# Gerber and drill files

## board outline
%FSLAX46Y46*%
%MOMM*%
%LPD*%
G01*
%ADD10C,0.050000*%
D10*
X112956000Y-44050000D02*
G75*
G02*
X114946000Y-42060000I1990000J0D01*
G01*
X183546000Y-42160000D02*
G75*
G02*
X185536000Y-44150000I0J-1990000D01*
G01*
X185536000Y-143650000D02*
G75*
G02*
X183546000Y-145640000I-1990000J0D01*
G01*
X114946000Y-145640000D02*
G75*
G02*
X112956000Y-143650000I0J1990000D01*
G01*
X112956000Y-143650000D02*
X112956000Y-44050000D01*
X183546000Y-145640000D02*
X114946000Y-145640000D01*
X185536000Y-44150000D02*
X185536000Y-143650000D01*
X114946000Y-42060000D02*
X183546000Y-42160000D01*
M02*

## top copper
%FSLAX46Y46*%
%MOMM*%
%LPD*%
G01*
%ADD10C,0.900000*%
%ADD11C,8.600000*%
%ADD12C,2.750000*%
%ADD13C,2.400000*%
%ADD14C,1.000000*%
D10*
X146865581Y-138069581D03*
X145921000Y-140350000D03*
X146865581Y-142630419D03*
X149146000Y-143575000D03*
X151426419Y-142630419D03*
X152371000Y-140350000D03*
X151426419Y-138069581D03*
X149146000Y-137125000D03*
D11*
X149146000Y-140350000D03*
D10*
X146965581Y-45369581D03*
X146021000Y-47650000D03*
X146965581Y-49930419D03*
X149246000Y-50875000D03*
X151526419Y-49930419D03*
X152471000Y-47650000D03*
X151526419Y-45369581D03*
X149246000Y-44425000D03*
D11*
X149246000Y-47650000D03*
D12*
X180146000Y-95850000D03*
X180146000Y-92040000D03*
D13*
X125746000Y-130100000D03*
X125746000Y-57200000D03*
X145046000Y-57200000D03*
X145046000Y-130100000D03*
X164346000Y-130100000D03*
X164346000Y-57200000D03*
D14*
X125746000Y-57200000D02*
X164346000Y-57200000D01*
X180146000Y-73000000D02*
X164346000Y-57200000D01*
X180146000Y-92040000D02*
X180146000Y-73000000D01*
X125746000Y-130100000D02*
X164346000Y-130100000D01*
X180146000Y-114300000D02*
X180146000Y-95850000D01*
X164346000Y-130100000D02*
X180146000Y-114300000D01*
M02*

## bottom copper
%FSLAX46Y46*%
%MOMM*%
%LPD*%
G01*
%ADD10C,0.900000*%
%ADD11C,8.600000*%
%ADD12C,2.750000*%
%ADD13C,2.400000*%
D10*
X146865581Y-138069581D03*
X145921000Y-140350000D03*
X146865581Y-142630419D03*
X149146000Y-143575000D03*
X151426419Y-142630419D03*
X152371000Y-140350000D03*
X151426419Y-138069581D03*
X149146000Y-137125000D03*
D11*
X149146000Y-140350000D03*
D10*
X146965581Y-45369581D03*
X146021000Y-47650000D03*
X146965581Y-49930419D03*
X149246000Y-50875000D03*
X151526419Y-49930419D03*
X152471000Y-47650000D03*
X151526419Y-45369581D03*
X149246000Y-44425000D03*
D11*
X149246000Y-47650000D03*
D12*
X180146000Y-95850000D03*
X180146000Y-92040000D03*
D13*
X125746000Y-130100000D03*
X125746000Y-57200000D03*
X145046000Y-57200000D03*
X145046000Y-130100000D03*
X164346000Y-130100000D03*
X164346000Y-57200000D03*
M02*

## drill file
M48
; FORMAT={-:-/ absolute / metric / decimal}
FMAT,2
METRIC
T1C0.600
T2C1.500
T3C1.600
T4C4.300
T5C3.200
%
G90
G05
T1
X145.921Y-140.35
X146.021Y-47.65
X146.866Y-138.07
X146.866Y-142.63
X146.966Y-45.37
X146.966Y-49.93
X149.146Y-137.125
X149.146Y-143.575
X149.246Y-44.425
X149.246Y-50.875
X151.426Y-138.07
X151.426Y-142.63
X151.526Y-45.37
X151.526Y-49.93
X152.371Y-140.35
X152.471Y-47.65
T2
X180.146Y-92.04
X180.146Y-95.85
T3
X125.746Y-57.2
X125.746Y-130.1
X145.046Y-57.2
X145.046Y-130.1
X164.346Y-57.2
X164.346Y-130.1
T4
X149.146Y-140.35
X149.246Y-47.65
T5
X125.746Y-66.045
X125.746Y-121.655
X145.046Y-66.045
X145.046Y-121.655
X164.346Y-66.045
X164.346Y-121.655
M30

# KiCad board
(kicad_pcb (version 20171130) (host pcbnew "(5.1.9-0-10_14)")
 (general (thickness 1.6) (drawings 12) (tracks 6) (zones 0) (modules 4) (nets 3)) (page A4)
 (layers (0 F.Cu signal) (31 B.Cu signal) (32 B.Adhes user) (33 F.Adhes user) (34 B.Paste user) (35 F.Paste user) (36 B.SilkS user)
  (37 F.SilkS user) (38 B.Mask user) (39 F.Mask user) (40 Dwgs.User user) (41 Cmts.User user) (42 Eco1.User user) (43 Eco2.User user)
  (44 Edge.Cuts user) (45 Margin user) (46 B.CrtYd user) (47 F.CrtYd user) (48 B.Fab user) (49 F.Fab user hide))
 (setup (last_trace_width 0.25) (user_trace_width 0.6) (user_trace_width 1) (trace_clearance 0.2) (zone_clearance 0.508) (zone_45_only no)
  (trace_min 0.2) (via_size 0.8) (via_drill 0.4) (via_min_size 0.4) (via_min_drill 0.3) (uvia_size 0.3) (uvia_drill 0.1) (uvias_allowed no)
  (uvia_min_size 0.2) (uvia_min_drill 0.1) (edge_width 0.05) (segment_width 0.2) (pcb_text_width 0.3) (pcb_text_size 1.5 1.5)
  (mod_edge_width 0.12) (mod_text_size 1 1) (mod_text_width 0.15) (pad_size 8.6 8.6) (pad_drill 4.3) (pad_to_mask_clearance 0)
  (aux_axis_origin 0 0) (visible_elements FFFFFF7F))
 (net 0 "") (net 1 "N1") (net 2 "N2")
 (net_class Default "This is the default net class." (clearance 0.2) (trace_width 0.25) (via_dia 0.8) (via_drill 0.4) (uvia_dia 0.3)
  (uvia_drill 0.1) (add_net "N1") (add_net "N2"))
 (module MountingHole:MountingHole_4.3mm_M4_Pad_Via (layer F.Cu) (at 149.146 140.35 90)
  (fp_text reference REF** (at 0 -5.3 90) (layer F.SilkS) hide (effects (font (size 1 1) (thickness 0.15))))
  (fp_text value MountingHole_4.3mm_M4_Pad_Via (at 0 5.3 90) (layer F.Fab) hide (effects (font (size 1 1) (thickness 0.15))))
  (pad 1 thru_hole circle (at 2.280419 -2.280419 90) (size 0.9 0.9) (drill 0.6) (layers *.Cu *.Mask))
  (pad 1 thru_hole circle (at 0 -3.225 90) (size 0.9 0.9) (drill 0.6) (layers *.Cu *.Mask))
  (pad 1 thru_hole circle (at -2.280419 -2.280419 90) (size 0.9 0.9) (drill 0.6) (layers *.Cu *.Mask))
  (pad 1 thru_hole circle (at -3.225 0 90) (size 0.9 0.9) (drill 0.6) (layers *.Cu *.Mask))
  (pad 1 thru_hole circle (at -2.280419 2.280419 90) (size 0.9 0.9) (drill 0.6) (layers *.Cu *.Mask))
  (pad 1 thru_hole circle (at 0 3.225 90) (size 0.9 0.9) (drill 0.6) (layers *.Cu *.Mask))
  (pad 1 thru_hole circle (at 2.280419 2.280419 90) (size 0.9 0.9) (drill 0.6) (layers *.Cu *.Mask))
  (pad 1 thru_hole circle (at 3.225 0 90) (size 0.9 0.9) (drill 0.6) (layers *.Cu *.Mask))
  (pad 1 thru_hole circle (at 0 0 90) (size 8.6 8.6) (drill 4.3) (layers *.Cu *.Mask)))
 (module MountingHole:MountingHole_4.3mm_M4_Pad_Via (layer F.Cu) (at 149.246 47.65 90)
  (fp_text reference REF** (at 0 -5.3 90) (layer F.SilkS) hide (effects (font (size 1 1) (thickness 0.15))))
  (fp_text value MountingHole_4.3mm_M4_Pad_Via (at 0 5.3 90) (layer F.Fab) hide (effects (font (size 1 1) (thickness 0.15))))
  (pad 1 thru_hole circle (at 2.280419 -2.280419 90) (size 0.9 0.9) (drill 0.6) (layers *.Cu *.Mask))
  (pad 1 thru_hole circle (at 0 -3.225 90) (size 0.9 0.9) (drill 0.6) (layers *.Cu *.Mask))
  (pad 1 thru_hole circle (at -2.280419 -2.280419 90) (size 0.9 0.9) (drill 0.6) (layers *.Cu *.Mask))
  (pad 1 thru_hole circle (at -3.225 0 90) (size 0.9 0.9) (drill 0.6) (layers *.Cu *.Mask))
  (pad 1 thru_hole circle (at -2.280419 2.280419 90) (size 0.9 0.9) (drill 0.6) (layers *.Cu *.Mask))
  (pad 1 thru_hole circle (at 0 3.225 90) (size 0.9 0.9) (drill 0.6) (layers *.Cu *.Mask))
  (pad 1 thru_hole circle (at 2.280419 2.280419 90) (size 0.9 0.9) (drill 0.6) (layers *.Cu *.Mask))
  (pad 1 thru_hole circle (at 3.225 0 90) (size 0.9 0.9) (drill 0.6) (layers *.Cu *.Mask))
  (pad 1 thru_hole circle (at 0 0 90) (size 8.6 8.6) (drill 4.3) (layers *.Cu *.Mask)))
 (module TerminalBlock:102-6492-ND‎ (layer F.Cu) (at 184.346 89.74 270)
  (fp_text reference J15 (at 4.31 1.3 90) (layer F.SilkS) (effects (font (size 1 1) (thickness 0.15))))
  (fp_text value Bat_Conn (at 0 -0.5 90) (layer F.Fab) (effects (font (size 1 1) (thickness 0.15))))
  (pad 2 thru_hole circle (at 6.11 4.2 270) (size 2.75 2.75) (drill 1.5) (layers *.Cu *.Mask) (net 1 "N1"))
  (pad 1 thru_hole circle (at 2.3 4.2 270) (size 2.75 2.75) (drill 1.5) (layers *.Cu *.Mask) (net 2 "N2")))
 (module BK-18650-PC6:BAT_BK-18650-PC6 (layer F.Cu) (at 145.046 93.85 270)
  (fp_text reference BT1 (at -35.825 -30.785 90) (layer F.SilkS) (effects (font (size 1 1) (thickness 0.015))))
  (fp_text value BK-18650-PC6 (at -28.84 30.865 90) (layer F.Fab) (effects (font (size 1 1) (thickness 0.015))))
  (pad None np_thru_hole circle (at 27.805 19.3 270) (size 3.2 3.2) (drill 3.2) (layers *.Cu *.Mask))
  (pad None np_thru_hole circle (at 27.805 -19.3 270) (size 3.2 3.2) (drill 3.2) (layers *.Cu *.Mask))
  (pad None np_thru_hole circle (at 27.805 0 270) (size 3.2 3.2) (drill 3.2) (layers *.Cu *.Mask))
  (pad None np_thru_hole circle (at -27.805 19.3 270) (size 3.2 3.2) (drill 3.2) (layers *.Cu *.Mask))
  (pad None np_thru_hole circle (at -27.805 -19.3 270) (size 3.2 3.2) (drill 3.2) (layers *.Cu *.Mask))
  (pad None np_thru_hole circle (at -27.805 0 270) (size 3.2 3.2) (drill 3.2) (layers *.Cu *.Mask))
  (pad 3 thru_hole circle (at 36.25 19.3 270) (size 2.4 2.4) (drill 1.6) (layers *.Cu *.Mask) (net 1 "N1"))
  (pad 3+ thru_hole circle (at -36.65 19.3 270) (size 2.4 2.4) (drill 1.6) (layers *.Cu *.Mask) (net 2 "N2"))
  (pad 2+ thru_hole circle (at -36.65 0 270) (size 2.4 2.4) (drill 1.6) (layers *.Cu *.Mask) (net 2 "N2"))
  (pad 2 thru_hole circle (at 36.25 0 270) (size 2.4 2.4) (drill 1.6) (layers *.Cu *.Mask) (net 1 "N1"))
  (pad 1 thru_hole circle (at 36.25 -19.3 270) (size 2.4 2.4) (drill 1.6) (layers *.Cu *.Mask) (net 1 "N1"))
  (pad 1+ thru_hole circle (at -36.65 -19.3 270) (size 2.4 2.4) (drill 1.6) (layers *.Cu *.Mask) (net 2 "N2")))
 (gr_arc (start 114.946 44.05) (end 114.946 42.06) (angle -90) (layer Edge.Cuts) (width 0.05))
 (gr_arc (start 183.546 44.15) (end 185.536 44.15) (angle -90) (layer Edge.Cuts) (width 0.05))
 (gr_arc (start 183.546 143.65) (end 183.546 145.64) (angle -90) (layer Edge.Cuts) (width 0.05))
 (gr_arc (start 114.946 143.65) (end 112.956 143.65) (angle -90) (layer Edge.Cuts) (width 0.05))
 (gr_line (start 112.956 143.65) (end 112.956 44.05) (layer Edge.Cuts) (width 0.05))
 (gr_line (start 183.546 145.64) (end 114.946 145.64) (layer Edge.Cuts) (width 0.05))
 (gr_line (start 185.536 44.15) (end 185.536 143.65) (layer Edge.Cuts) (width 0.05))
 (gr_line (start 114.946 42.06) (end 183.546 42.16) (layer Edge.Cuts) (width 0.05))
 (segment (start 125.746 57.2) (end 164.346 57.2) (width 1) (layer F.Cu) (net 2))
 (segment (start 180.146 73) (end 164.346 57.2) (width 1) (layer F.Cu) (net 2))
 (segment (start 180.146 92.04) (end 180.146 73) (width 1) (layer F.Cu) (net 2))
 (segment (start 125.746 130.1) (end 164.346 130.1) (width 1) (layer F.Cu) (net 1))
 (segment (start 180.146 114.3) (end 180.146 95.85) (width 1) (layer F.Cu) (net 1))
 (segment (start 164.346 130.1) (end 180.146 114.3) (width 1) (layer F.Cu) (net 1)))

